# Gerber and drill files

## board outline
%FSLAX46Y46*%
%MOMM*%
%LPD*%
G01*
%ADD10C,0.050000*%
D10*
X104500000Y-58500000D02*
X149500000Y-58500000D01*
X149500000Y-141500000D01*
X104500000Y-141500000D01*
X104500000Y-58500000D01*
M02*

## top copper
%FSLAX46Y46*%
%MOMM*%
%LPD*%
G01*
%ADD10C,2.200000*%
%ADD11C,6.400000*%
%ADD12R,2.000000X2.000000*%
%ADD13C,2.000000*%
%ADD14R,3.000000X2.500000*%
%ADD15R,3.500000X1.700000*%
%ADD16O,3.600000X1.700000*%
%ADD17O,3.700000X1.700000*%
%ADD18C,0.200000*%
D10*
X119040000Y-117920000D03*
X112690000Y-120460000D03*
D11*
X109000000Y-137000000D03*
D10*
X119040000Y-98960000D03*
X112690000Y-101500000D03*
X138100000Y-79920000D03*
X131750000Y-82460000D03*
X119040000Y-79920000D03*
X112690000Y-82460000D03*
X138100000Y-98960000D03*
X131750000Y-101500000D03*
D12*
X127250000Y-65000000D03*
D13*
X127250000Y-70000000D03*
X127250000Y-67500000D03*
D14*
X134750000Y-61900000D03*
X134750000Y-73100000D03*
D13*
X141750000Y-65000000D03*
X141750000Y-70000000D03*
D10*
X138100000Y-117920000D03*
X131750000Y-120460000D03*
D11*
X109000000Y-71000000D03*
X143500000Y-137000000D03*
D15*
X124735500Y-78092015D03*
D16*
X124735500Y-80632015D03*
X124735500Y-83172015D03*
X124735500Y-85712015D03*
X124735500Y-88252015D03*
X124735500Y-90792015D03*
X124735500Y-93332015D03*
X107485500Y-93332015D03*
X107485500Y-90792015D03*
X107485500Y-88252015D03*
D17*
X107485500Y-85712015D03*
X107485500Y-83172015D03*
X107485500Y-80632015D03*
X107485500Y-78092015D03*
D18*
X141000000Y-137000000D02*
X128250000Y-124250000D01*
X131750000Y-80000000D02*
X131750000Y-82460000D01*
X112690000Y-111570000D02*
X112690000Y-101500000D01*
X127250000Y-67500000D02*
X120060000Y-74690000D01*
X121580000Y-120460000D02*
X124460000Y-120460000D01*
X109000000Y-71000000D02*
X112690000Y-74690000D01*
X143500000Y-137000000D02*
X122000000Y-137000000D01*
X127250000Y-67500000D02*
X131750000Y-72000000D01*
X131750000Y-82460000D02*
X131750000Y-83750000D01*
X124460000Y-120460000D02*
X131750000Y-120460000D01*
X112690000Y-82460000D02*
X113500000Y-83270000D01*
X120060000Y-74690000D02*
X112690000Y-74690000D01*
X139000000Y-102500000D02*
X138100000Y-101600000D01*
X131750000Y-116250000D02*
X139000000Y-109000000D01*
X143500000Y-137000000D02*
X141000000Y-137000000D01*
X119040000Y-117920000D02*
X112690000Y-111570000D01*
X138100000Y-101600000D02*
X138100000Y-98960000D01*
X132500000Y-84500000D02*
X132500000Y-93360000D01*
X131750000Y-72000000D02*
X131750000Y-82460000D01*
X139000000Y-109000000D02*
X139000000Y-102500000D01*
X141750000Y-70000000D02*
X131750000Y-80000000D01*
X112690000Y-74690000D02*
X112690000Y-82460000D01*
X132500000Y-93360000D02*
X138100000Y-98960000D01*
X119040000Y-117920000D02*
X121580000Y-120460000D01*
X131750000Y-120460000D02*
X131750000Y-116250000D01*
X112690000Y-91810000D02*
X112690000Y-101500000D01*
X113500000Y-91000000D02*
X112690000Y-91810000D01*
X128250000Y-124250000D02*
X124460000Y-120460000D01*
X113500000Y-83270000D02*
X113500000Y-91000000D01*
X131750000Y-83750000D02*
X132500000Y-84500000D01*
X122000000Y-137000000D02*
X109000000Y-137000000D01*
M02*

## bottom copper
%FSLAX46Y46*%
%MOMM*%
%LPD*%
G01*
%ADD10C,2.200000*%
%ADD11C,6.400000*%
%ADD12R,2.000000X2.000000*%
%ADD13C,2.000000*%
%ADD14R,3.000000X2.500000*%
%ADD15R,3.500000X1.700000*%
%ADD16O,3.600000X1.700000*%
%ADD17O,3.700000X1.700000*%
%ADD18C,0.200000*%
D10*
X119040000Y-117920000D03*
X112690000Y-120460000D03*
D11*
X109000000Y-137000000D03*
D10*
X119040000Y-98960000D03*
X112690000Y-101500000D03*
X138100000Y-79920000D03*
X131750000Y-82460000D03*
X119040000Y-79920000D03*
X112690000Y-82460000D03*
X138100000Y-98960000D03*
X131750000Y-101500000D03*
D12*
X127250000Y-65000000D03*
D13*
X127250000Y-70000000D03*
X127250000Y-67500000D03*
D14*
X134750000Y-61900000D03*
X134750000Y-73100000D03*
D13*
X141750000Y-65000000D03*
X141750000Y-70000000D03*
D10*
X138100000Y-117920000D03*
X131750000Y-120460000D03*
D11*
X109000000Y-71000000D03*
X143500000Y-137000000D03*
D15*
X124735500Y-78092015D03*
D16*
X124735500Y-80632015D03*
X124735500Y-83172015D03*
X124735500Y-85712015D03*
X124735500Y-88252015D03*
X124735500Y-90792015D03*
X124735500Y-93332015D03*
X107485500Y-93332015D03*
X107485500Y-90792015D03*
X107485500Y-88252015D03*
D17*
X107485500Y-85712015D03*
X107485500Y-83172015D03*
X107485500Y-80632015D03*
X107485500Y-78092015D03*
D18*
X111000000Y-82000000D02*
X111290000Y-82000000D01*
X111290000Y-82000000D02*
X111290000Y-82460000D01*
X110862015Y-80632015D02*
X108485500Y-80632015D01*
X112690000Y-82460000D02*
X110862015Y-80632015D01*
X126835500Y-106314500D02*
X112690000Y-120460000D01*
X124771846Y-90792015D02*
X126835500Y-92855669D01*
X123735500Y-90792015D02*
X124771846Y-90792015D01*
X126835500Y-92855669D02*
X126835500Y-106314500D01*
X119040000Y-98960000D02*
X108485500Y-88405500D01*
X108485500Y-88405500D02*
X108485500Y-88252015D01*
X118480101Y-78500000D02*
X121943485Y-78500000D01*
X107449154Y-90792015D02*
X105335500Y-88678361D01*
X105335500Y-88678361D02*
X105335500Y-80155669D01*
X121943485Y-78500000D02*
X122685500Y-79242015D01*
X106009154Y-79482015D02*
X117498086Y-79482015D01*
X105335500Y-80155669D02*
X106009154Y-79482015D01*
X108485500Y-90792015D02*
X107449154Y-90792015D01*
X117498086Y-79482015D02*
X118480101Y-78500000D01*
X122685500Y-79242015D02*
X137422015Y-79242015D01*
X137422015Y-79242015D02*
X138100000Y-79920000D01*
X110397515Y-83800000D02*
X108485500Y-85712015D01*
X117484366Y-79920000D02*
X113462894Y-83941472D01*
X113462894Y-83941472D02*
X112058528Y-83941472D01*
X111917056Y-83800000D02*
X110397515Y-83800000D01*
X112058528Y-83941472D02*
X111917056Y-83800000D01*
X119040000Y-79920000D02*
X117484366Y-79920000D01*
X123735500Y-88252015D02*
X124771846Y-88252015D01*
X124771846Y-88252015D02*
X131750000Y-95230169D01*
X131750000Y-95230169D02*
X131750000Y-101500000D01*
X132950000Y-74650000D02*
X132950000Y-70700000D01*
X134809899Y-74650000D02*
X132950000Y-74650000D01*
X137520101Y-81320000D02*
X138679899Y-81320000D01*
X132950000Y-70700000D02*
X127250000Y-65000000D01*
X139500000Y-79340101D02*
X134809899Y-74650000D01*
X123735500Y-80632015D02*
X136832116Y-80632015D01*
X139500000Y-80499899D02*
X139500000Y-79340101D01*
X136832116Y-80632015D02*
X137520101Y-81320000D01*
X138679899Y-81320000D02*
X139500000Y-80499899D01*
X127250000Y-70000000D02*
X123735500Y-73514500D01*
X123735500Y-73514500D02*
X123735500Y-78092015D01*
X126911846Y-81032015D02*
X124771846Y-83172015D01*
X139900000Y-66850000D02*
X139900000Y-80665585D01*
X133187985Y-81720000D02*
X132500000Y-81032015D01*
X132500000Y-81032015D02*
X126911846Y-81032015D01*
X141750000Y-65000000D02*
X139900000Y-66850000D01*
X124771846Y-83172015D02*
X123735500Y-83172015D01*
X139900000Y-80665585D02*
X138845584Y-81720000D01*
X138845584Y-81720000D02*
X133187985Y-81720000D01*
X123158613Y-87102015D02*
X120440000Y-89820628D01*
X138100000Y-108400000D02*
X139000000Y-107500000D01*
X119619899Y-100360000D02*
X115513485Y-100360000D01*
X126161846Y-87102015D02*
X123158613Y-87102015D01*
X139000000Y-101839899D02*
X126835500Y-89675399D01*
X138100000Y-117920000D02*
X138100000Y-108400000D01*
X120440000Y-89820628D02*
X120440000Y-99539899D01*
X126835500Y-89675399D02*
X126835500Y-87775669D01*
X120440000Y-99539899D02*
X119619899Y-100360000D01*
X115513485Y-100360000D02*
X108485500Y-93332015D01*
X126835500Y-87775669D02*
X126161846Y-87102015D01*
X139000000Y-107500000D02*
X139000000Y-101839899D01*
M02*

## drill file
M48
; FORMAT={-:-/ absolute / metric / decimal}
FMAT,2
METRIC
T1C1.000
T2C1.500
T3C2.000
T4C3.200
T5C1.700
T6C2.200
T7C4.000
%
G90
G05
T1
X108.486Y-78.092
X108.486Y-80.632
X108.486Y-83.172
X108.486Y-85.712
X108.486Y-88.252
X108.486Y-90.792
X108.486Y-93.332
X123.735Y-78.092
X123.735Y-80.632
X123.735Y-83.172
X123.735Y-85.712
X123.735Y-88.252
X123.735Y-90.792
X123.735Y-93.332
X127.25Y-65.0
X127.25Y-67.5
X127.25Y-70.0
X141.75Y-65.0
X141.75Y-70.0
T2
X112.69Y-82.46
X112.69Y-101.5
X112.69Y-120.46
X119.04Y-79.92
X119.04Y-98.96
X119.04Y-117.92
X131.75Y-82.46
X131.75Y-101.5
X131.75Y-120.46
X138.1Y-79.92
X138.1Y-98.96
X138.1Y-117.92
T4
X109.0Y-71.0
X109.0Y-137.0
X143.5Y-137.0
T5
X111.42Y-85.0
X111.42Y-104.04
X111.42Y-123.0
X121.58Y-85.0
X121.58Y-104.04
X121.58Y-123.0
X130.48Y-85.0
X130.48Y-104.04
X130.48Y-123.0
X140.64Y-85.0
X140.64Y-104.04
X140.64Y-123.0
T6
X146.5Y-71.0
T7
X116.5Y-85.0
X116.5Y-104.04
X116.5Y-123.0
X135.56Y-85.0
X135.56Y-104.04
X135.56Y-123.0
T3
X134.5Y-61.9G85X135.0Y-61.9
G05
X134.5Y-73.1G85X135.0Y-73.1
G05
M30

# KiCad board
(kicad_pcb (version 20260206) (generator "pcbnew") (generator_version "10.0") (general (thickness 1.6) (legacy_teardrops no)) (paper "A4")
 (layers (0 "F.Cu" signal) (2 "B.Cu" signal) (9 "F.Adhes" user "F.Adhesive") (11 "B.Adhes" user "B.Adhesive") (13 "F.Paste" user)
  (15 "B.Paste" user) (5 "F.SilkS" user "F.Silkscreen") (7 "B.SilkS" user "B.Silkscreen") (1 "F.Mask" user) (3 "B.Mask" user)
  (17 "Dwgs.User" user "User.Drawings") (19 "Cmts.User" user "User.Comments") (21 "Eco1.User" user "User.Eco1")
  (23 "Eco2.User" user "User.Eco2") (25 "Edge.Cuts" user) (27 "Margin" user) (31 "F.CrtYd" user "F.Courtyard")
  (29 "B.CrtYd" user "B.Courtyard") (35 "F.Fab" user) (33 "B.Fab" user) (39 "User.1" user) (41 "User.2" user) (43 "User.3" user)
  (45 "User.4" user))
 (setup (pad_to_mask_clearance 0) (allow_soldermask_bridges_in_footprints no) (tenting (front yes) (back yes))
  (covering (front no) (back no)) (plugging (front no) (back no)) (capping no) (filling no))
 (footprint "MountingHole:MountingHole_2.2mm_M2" (layer "F.Cu") (at 146.5 71)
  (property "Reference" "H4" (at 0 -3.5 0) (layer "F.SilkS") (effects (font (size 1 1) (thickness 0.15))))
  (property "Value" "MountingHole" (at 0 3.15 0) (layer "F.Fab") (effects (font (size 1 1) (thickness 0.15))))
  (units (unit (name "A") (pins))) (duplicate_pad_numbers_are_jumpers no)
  (pad "" np_thru_hole circle (at 0 0) (size 2.2 2.2) (drill 2.2) (layers "*.Cu" "*.Mask")))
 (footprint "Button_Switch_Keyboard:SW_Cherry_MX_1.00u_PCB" (layer "F.Cu") (at 119.04 117.92)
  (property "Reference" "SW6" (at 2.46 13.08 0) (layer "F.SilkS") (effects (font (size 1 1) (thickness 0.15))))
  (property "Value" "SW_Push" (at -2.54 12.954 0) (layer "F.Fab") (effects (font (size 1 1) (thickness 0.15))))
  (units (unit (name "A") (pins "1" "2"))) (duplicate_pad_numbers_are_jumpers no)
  (pad "" np_thru_hole circle (at -7.62 5.08) (size 1.7 1.7) (drill 1.7) (layers "*.Cu" "*.Mask"))
  (pad "" np_thru_hole circle (at -2.54 5.08) (size 4 4) (drill 4) (layers "*.Cu" "*.Mask"))
  (pad "" np_thru_hole circle (at 2.54 5.08) (size 1.7 1.7) (drill 1.7) (layers "*.Cu" "*.Mask"))
  (pad "1" thru_hole circle (at 0 0) (size 2.2 2.2) (drill 1.5) (layers "*.Cu" "*.Mask") (remove_unused_layers no) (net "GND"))
  (pad "2" thru_hole circle (at -6.35 2.54) (size 2.2 2.2) (drill 1.5) (layers "*.Cu" "*.Mask") (remove_unused_layers no)
   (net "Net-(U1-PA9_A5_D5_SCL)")))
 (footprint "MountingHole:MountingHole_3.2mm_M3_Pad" (layer "F.Cu") (at 109 137)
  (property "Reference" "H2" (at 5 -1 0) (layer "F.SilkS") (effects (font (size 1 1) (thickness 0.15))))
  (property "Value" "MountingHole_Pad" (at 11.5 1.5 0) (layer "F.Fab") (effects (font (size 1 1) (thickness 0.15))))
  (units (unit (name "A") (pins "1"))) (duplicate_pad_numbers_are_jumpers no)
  (pad "1" thru_hole circle (at 0 0) (size 6.4 6.4) (drill 3.2) (layers "*.Cu" "*.Mask") (remove_unused_layers no) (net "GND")
   (zone_connect 2)))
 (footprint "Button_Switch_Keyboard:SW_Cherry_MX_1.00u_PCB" (layer "F.Cu") (at 119.04 98.96)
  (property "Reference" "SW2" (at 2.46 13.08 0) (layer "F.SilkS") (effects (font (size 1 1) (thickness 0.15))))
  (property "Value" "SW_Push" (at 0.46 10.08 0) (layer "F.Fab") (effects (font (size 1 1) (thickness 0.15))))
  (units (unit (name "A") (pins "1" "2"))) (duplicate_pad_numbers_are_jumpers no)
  (pad "" np_thru_hole circle (at -7.62 5.08) (size 1.7 1.7) (drill 1.7) (layers "*.Cu" "*.Mask"))
  (pad "" np_thru_hole circle (at -2.54 5.08) (size 4 4) (drill 4) (layers "*.Cu" "*.Mask"))
  (pad "" np_thru_hole circle (at 2.54 5.08) (size 1.7 1.7) (drill 1.7) (layers "*.Cu" "*.Mask"))
  (pad "1" thru_hole circle (at 0 0) (size 2.2 2.2) (drill 1.5) (layers "*.Cu" "*.Mask") (remove_unused_layers no)
   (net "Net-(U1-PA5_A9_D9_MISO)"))
  (pad "2" thru_hole circle (at -6.35 2.54) (size 2.2 2.2) (drill 1.5) (layers "*.Cu" "*.Mask") (remove_unused_layers no) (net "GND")))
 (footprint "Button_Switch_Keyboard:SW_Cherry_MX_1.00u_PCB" (layer "F.Cu") (at 138.1 79.92)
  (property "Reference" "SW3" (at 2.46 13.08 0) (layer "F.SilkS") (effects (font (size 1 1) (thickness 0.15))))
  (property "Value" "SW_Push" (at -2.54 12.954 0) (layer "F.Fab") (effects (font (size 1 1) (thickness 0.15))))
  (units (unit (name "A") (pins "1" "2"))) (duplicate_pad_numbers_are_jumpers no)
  (pad "" np_thru_hole circle (at -7.62 5.08) (size 1.7 1.7) (drill 1.7) (layers "*.Cu" "*.Mask"))
  (pad "" np_thru_hole circle (at -2.54 5.08) (size 4 4) (drill 4) (layers "*.Cu" "*.Mask"))
  (pad "" np_thru_hole circle (at 2.54 5.08) (size 1.7 1.7) (drill 1.7) (layers "*.Cu" "*.Mask"))
  (pad "1" thru_hole circle (at 0 0) (size 2.2 2.2) (drill 1.5) (layers "*.Cu" "*.Mask") (remove_unused_layers no)
   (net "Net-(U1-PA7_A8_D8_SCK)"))
  (pad "2" thru_hole circle (at -6.35 2.54) (size 2.2 2.2) (drill 1.5) (layers "*.Cu" "*.Mask") (remove_unused_layers no) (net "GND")))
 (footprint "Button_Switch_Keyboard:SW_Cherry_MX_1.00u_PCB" (layer "F.Cu") (at 119.04 79.92)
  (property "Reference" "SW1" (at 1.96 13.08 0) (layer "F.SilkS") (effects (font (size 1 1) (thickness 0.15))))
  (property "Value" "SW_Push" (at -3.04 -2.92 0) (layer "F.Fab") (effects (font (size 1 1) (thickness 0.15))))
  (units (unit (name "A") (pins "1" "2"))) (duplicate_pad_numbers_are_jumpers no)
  (pad "" np_thru_hole circle (at -7.62 5.08) (size 1.7 1.7) (drill 1.7) (layers "*.Cu" "*.Mask"))
  (pad "" np_thru_hole circle (at -2.54 5.08) (size 4 4) (drill 4) (layers "*.Cu" "*.Mask"))
  (pad "" np_thru_hole circle (at 2.54 5.08) (size 1.7 1.7) (drill 1.7) (layers "*.Cu" "*.Mask"))
  (pad "1" thru_hole circle (at 0 0) (size 2.2 2.2) (drill 1.5) (layers "*.Cu" "*.Mask") (remove_unused_layers no)
   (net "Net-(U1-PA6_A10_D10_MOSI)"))
  (pad "2" thru_hole circle (at -6.35 2.54) (size 2.2 2.2) (drill 1.5) (layers "*.Cu" "*.Mask") (remove_unused_layers no) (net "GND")))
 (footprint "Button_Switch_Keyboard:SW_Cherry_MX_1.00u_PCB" (layer "F.Cu") (at 138.1 98.96)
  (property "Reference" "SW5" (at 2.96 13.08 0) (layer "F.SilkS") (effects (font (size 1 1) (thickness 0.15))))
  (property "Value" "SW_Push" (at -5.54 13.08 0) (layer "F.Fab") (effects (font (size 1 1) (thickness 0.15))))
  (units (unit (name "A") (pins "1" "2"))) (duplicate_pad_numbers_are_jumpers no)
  (pad "" np_thru_hole circle (at -7.62 5.08) (size 1.7 1.7) (drill 1.7) (layers "*.Cu" "*.Mask"))
  (pad "" np_thru_hole circle (at -2.54 5.08) (size 4 4) (drill 4) (layers "*.Cu" "*.Mask"))
  (pad "" np_thru_hole circle (at 2.54 5.08) (size 1.7 1.7) (drill 1.7) (layers "*.Cu" "*.Mask"))
  (pad "1" thru_hole circle (at 0 0) (size 2.2 2.2) (drill 1.5) (layers "*.Cu" "*.Mask") (remove_unused_layers no) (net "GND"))
  (pad "2" thru_hole circle (at -6.35 2.54) (size 2.2 2.2) (drill 1.5) (layers "*.Cu" "*.Mask") (remove_unused_layers no)
   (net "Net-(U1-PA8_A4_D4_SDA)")))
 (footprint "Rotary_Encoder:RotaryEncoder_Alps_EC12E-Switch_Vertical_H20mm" (layer "F.Cu") (at 127.25 65)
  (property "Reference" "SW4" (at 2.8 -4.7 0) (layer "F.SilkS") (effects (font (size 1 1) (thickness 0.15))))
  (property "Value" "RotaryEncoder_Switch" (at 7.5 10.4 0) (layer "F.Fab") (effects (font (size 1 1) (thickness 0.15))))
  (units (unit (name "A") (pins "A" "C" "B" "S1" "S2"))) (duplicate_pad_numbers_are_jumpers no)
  (pad "A" thru_hole rect (at 0 0) (size 2 2) (drill 1) (layers "*.Cu" "*.Mask") (remove_unused_layers no) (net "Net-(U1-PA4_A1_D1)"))
  (pad "B" thru_hole circle (at 0 5) (size 2 2) (drill 1) (layers "*.Cu" "*.Mask") (remove_unused_layers no) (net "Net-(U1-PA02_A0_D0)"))
  (pad "C" thru_hole circle (at 0 2.5) (size 2 2) (drill 1) (layers "*.Cu" "*.Mask") (remove_unused_layers no) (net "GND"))
  (pad "MP" thru_hole rect (at 7.5 -3.1) (size 3 2.5) (drill oval 2.5 2) (layers "*.Cu" "*.Mask") (remove_unused_layers no))
  (pad "MP" thru_hole rect (at 7.5 8.1) (size 3 2.5) (drill oval 2.5 2) (layers "*.Cu" "*.Mask") (remove_unused_layers no))
  (pad "S1" thru_hole circle (at 14.5 0) (size 2 2) (drill 1) (layers "*.Cu" "*.Mask") (remove_unused_layers no) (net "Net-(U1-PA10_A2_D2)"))
  (pad "S2" thru_hole circle (at 14.5 5) (size 2 2) (drill 1) (layers "*.Cu" "*.Mask") (remove_unused_layers no) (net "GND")))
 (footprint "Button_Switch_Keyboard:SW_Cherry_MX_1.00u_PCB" (layer "F.Cu") (at 138.1 117.92)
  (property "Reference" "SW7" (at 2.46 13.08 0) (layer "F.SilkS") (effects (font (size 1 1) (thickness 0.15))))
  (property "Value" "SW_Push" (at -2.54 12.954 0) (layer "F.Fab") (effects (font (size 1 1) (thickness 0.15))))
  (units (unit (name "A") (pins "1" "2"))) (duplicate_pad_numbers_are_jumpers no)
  (pad "" np_thru_hole circle (at -7.62 5.08) (size 1.7 1.7) (drill 1.7) (layers "*.Cu" "*.Mask"))
  (pad "" np_thru_hole circle (at -2.54 5.08) (size 4 4) (drill 4) (layers "*.Cu" "*.Mask"))
  (pad "" np_thru_hole circle (at 2.54 5.08) (size 1.7 1.7) (drill 1.7) (layers "*.Cu" "*.Mask"))
  (pad "1" thru_hole circle (at 0 0) (size 2.2 2.2) (drill 1.5) (layers "*.Cu" "*.Mask") (remove_unused_layers no)
   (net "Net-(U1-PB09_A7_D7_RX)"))
  (pad "2" thru_hole circle (at -6.35 2.54) (size 2.2 2.2) (drill 1.5) (layers "*.Cu" "*.Mask") (remove_unused_layers no) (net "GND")))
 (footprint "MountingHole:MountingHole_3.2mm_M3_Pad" (layer "F.Cu") (at 109 71)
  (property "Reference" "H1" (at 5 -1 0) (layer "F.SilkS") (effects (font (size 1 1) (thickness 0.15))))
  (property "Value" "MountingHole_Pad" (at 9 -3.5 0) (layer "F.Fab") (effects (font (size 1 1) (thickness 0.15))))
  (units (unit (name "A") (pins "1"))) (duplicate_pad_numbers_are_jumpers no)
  (pad "1" thru_hole circle (at 0 0) (size 6.4 6.4) (drill 3.2) (layers "*.Cu" "*.Mask") (remove_unused_layers no) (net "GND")
   (zone_connect 2)))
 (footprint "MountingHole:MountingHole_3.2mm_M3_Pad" (layer "F.Cu") (at 143.5 137)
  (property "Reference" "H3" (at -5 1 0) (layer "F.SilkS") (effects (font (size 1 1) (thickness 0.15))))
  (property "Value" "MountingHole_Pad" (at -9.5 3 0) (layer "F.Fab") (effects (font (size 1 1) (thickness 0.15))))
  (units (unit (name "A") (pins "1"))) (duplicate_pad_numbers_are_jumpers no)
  (pad "1" thru_hole circle (at 0 0) (size 6.4 6.4) (drill 3.2) (layers "*.Cu" "*.Mask") (remove_unused_layers no) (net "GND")
   (zone_connect 2)))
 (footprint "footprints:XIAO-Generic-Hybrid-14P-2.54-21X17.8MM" (layer "B.Cu") (at 116.1105 85.712015 180)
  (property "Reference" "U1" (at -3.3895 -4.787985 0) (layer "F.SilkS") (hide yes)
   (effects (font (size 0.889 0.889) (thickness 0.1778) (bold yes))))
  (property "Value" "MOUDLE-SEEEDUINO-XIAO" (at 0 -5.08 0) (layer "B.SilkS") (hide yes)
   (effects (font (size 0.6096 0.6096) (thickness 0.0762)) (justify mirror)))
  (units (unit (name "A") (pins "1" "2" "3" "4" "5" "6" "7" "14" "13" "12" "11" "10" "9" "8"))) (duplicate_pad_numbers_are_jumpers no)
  (pad "1" thru_hole rect (at -7.625 7.62 180) (size 3.5 1.7) (drill 1 (offset -1 0)) (layers "*.Cu" "*.Mask") (remove_unused_layers no)
   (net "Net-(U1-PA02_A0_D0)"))
  (pad "2" thru_hole oval (at -7.625 5.08 180) (size 3.6 1.7) (drill 1 (offset -1 0)) (layers "*.Cu" "*.Mask") (remove_unused_layers no)
   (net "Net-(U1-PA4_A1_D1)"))
  (pad "3" thru_hole oval (at -7.625 2.54 180) (size 3.6 1.7) (drill 1 (offset -1 0)) (layers "*.Cu" "*.Mask") (remove_unused_layers no)
   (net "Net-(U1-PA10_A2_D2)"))
  (pad "4" thru_hole oval (at -7.625 0 180) (size 3.6 1.7) (drill 1 (offset -1 0)) (layers "*.Cu" "*.Mask") (remove_unused_layers no)
   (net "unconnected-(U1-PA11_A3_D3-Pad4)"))
  (pad "5" thru_hole oval (at -7.625 -2.54 180) (size 3.6 1.7) (drill 1 (offset -1 0)) (layers "*.Cu" "*.Mask") (remove_unused_layers no)
   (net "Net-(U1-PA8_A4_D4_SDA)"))
  (pad "6" thru_hole oval (at -7.625 -5.08) (size 3.6 1.7) (drill 1 (offset 1 0)) (layers "*.Cu" "*.Mask") (remove_unused_layers no)
   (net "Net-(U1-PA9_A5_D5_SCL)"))
  (pad "7" thru_hole oval (at -7.625 -7.62 180) (size 3.6 1.7) (drill 1 (offset -1 0)) (layers "*.Cu" "*.Mask") (remove_unused_layers no)
   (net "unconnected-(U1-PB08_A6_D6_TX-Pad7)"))
  (pad "8" thru_hole oval (at 7.625 -7.62 180) (size 3.6 1.7) (drill 1 (offset 1 0)) (layers "*.Cu" "*.Mask") (remove_unused_layers no)
   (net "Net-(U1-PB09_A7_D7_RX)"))
  (pad "9" thru_hole oval (at 7.625 -5.08 180) (size 3.6 1.7) (drill 1 (offset 1 0)) (layers "*.Cu" "*.Mask") (remove_unused_layers no)
   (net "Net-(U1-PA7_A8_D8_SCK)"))
  (pad "10" thru_hole oval (at 7.625 -2.54 180) (size 3.6 1.7) (drill 1 (offset 1 0)) (layers "*.Cu" "*.Mask") (remove_unused_layers no)
   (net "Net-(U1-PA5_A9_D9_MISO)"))
  (pad "11" thru_hole oval (at 7.625 0 180) (size 3.7 1.7) (drill 1 (offset 1 0)) (layers "*.Cu" "*.Mask") (remove_unused_layers no)
   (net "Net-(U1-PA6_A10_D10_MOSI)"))
  (pad "12" thru_hole oval (at 7.625 2.54 180) (size 3.7 1.7) (drill 1 (offset 1 0)) (layers "*.Cu" "*.Mask") (remove_unused_layers no)
   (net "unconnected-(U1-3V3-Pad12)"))
  (pad "13" thru_hole oval (at 7.625 5.08 180) (size 3.7 1.7) (drill 1 (offset 1 0)) (layers "*.Cu" "*.Mask") (remove_unused_layers no)
   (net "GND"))
  (pad "14" thru_hole oval (at 7.625 7.62 180) (size 3.7 1.7) (drill 1 (offset 1 0)) (layers "*.Cu" "*.Mask") (remove_unused_layers no)
   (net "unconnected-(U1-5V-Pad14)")))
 (gr_rect (start 104.5 58.5) (end 149.5 141.5) (stroke (width 0.05) (type default)) (fill no) (layer "Edge.Cuts"))
 (segment (start 111 82) (end 111.29 82) (width 0.2) (layer "B.Cu") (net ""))
 (segment (start 111.29 82) (end 111.29 82.46) (width 0.2) (layer "B.Cu") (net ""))
 (segment (start 141 137) (end 128.25 124.25) (width 0.2) (layer "F.Cu") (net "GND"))
 (segment (start 131.75 80) (end 131.75 82.46) (width 0.2) (layer "F.Cu") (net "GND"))
 (segment (start 112.69 111.57) (end 112.69 101.5) (width 0.2) (layer "F.Cu") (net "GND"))
 (segment (start 127.25 67.5) (end 120.06 74.69) (width 0.2) (layer "F.Cu") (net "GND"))
 (segment (start 121.58 120.46) (end 124.46 120.46) (width 0.2) (layer "F.Cu") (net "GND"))
 (segment (start 109 71) (end 112.69 74.69) (width 0.2) (layer "F.Cu") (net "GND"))
 (segment (start 143.5 137) (end 122 137) (width 0.2) (layer "F.Cu") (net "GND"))
 (segment (start 127.25 67.5) (end 131.75 72) (width 0.2) (layer "F.Cu") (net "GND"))
 (segment (start 131.75 82.46) (end 131.75 83.75) (width 0.2) (layer "F.Cu") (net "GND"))
 (segment (start 124.46 120.46) (end 131.75 120.46) (width 0.2) (layer "F.Cu") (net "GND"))
 (segment (start 112.69 82.46) (end 113.5 83.27) (width 0.2) (layer "F.Cu") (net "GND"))
 (segment (start 120.06 74.69) (end 112.69 74.69) (width 0.2) (layer "F.Cu") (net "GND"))
 (segment (start 139 102.5) (end 138.1 101.6) (width 0.2) (layer "F.Cu") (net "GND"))
 (segment (start 131.75 116.25) (end 139 109) (width 0.2) (layer "F.Cu") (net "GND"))
 (segment (start 143.5 137) (end 141 137) (width 0.2) (layer "F.Cu") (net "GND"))
 (segment (start 119.04 117.92) (end 112.69 111.57) (width 0.2) (layer "F.Cu") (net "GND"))
 (segment (start 138.1 101.6) (end 138.1 98.96) (width 0.2) (layer "F.Cu") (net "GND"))
 (segment (start 132.5 84.5) (end 132.5 93.36) (width 0.2) (layer "F.Cu") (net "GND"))
 (segment (start 131.75 72) (end 131.75 82.46) (width 0.2) (layer "F.Cu") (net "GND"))
 (segment (start 139 109) (end 139 102.5) (width 0.2) (layer "F.Cu") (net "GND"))
 (segment (start 141.75 70) (end 131.75 80) (width 0.2) (layer "F.Cu") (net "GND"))
 (segment (start 112.69 74.69) (end 112.69 82.46) (width 0.2) (layer "F.Cu") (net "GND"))
 (segment (start 132.5 93.36) (end 138.1 98.96) (width 0.2) (layer "F.Cu") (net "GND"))
 (segment (start 119.04 117.92) (end 121.58 120.46) (width 0.2) (layer "F.Cu") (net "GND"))
 (segment (start 131.75 120.46) (end 131.75 116.25) (width 0.2) (layer "F.Cu") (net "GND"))
 (segment (start 112.69 91.81) (end 112.69 101.5) (width 0.2) (layer "F.Cu") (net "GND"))
 (segment (start 113.5 91) (end 112.69 91.81) (width 0.2) (layer "F.Cu") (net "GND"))
 (segment (start 128.25 124.25) (end 124.46 120.46) (width 0.2) (layer "F.Cu") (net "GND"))
 (segment (start 113.5 83.27) (end 113.5 91) (width 0.2) (layer "F.Cu") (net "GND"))
 (segment (start 131.75 83.75) (end 132.5 84.5) (width 0.2) (layer "F.Cu") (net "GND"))
 (segment (start 122 137) (end 109 137) (width 0.2) (layer "F.Cu") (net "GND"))
 (segment (start 110.862015 80.632015) (end 108.4855 80.632015) (width 0.2) (layer "B.Cu") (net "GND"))
 (segment (start 112.69 82.46) (end 110.862015 80.632015) (width 0.2) (layer "B.Cu") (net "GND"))
 (segment (start 126.8355 106.3145) (end 112.69 120.46) (width 0.2) (layer "B.Cu") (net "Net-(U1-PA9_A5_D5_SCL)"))
 (segment (start 124.771846 90.792015) (end 126.8355 92.855669) (width 0.2) (layer "B.Cu") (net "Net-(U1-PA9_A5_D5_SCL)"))
 (segment (start 123.7355 90.792015) (end 124.771846 90.792015) (width 0.2) (layer "B.Cu") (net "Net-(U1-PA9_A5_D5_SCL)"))
 (segment (start 126.8355 92.855669) (end 126.8355 106.3145) (width 0.2) (layer "B.Cu") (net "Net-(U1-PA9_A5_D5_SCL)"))
 (segment (start 119.04 98.96) (end 108.4855 88.4055) (width 0.2) (layer "B.Cu") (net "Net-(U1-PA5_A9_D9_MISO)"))
 (segment (start 108.4855 88.4055) (end 108.4855 88.252015) (width 0.2) (layer "B.Cu") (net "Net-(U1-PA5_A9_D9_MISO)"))
 (segment (start 118.480101 78.5) (end 121.943485 78.5) (width 0.2) (layer "B.Cu") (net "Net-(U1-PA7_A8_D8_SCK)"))
 (segment (start 107.449154 90.792015) (end 105.3355 88.678361) (width 0.2) (layer "B.Cu") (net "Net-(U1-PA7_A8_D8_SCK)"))
 (segment (start 105.3355 88.678361) (end 105.3355 80.155669) (width 0.2) (layer "B.Cu") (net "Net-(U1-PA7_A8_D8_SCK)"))
 (segment (start 121.943485 78.5) (end 122.6855 79.242015) (width 0.2) (layer "B.Cu") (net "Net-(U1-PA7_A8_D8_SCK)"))
 (segment (start 106.009154 79.482015) (end 117.498086 79.482015) (width 0.2) (layer "B.Cu") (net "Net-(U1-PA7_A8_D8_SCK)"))
 (segment (start 105.3355 80.155669) (end 106.009154 79.482015) (width 0.2) (layer "B.Cu") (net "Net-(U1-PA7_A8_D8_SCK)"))
 (segment (start 108.4855 90.792015) (end 107.449154 90.792015) (width 0.2) (layer "B.Cu") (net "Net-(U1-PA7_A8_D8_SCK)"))
 (segment (start 117.498086 79.482015) (end 118.480101 78.5) (width 0.2) (layer "B.Cu") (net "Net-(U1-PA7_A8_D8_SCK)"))
 (segment (start 122.6855 79.242015) (end 137.422015 79.242015) (width 0.2) (layer "B.Cu") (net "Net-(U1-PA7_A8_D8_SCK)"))
 (segment (start 137.422015 79.242015) (end 138.1 79.92) (width 0.2) (layer "B.Cu") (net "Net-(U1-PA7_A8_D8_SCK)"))
 (segment (start 110.397515 83.8) (end 108.4855 85.712015) (width 0.2) (layer "B.Cu") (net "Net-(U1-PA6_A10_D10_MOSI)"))
 (segment (start 117.484366 79.92) (end 113.462894 83.941472) (width 0.2) (layer "B.Cu") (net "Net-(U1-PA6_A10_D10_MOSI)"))
 (segment (start 113.462894 83.941472) (end 112.058528 83.941472) (width 0.2) (layer "B.Cu") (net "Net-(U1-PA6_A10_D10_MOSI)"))
 (segment (start 111.917056 83.8) (end 110.397515 83.8) (width 0.2) (layer "B.Cu") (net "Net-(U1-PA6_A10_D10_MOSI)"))
 (segment (start 112.058528 83.941472) (end 111.917056 83.8) (width 0.2) (layer "B.Cu") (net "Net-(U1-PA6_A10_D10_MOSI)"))
 (segment (start 119.04 79.92) (end 117.484366 79.92) (width 0.2) (layer "B.Cu") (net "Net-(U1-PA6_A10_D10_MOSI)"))
 (segment (start 123.7355 88.252015) (end 124.771846 88.252015) (width 0.2) (layer "B.Cu") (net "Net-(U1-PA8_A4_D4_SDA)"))
 (segment (start 124.771846 88.252015) (end 131.75 95.230169) (width 0.2) (layer "B.Cu") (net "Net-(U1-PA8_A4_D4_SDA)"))
 (segment (start 131.75 95.230169) (end 131.75 101.5) (width 0.2) (layer "B.Cu") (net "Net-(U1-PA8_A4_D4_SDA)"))
 (segment (start 132.95 74.65) (end 132.95 70.7) (width 0.2) (layer "B.Cu") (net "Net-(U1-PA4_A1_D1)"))
 (segment (start 134.809899 74.65) (end 132.95 74.65) (width 0.2) (layer "B.Cu") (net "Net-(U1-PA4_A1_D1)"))
 (segment (start 137.520101 81.32) (end 138.679899 81.32) (width 0.2) (layer "B.Cu") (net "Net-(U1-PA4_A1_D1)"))
 (segment (start 132.95 70.7) (end 127.25 65) (width 0.2) (layer "B.Cu") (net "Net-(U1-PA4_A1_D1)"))
 (segment (start 139.5 79.340101) (end 134.809899 74.65) (width 0.2) (layer "B.Cu") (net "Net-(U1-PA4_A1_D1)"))
 (segment (start 123.7355 80.632015) (end 136.832116 80.632015) (width 0.2) (layer "B.Cu") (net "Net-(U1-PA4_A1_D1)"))
 (segment (start 139.5 80.499899) (end 139.5 79.340101) (width 0.2) (layer "B.Cu") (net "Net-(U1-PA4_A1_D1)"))
 (segment (start 136.832116 80.632015) (end 137.520101 81.32) (width 0.2) (layer "B.Cu") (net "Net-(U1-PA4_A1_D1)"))
 (segment (start 138.679899 81.32) (end 139.5 80.499899) (width 0.2) (layer "B.Cu") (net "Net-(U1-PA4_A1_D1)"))
 (segment (start 127.25 70) (end 123.7355 73.5145) (width 0.2) (layer "B.Cu") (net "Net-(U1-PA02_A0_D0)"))
 (segment (start 123.7355 73.5145) (end 123.7355 78.092015) (width 0.2) (layer "B.Cu") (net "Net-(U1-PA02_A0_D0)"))
 (segment (start 126.911846 81.032015) (end 124.771846 83.172015) (width 0.2) (layer "B.Cu") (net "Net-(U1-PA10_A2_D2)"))
 (segment (start 139.9 66.85) (end 139.9 80.665585) (width 0.2) (layer "B.Cu") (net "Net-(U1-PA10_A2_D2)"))
 (segment (start 133.187985 81.72) (end 132.5 81.032015) (width 0.2) (layer "B.Cu") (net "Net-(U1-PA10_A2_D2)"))
 (segment (start 132.5 81.032015) (end 126.911846 81.032015) (width 0.2) (layer "B.Cu") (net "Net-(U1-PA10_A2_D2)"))
 (segment (start 141.75 65) (end 139.9 66.85) (width 0.2) (layer "B.Cu") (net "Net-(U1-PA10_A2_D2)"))
 (segment (start 124.771846 83.172015) (end 123.7355 83.172015) (width 0.2) (layer "B.Cu") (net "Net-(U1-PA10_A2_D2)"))
 (segment (start 139.9 80.665585) (end 138.845584 81.72) (width 0.2) (layer "B.Cu") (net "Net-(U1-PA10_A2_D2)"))
 (segment (start 138.845584 81.72) (end 133.187985 81.72) (width 0.2) (layer "B.Cu") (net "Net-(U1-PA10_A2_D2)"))
 (segment (start 123.158613 87.102015) (end 120.44 89.820628) (width 0.2) (layer "B.Cu") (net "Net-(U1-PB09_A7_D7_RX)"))
 (segment (start 138.1 108.4) (end 139 107.5) (width 0.2) (layer "B.Cu") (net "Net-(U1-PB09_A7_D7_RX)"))
 (segment (start 119.619899 100.36) (end 115.513485 100.36) (width 0.2) (layer "B.Cu") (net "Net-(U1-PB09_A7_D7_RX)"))
 (segment (start 126.161846 87.102015) (end 123.158613 87.102015) (width 0.2) (layer "B.Cu") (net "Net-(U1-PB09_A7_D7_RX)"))
 (segment (start 139 101.839899) (end 126.8355 89.675399) (width 0.2) (layer "B.Cu") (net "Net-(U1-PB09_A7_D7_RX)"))
 (segment (start 138.1 117.92) (end 138.1 108.4) (width 0.2) (layer "B.Cu") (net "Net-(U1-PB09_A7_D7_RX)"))
 (segment (start 120.44 89.820628) (end 120.44 99.539899) (width 0.2) (layer "B.Cu") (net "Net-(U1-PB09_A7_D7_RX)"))
 (segment (start 126.8355 89.675399) (end 126.8355 87.775669) (width 0.2) (layer "B.Cu") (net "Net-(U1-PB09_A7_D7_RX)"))
 (segment (start 120.44 99.539899) (end 119.619899 100.36) (width 0.2) (layer "B.Cu") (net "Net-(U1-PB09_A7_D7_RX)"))
 (segment (start 115.513485 100.36) (end 108.4855 93.332015) (width 0.2) (layer "B.Cu") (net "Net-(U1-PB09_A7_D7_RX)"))
 (segment (start 126.8355 87.775669) (end 126.161846 87.102015) (width 0.2) (layer "B.Cu") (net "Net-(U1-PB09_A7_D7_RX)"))
 (segment (start 139 107.5) (end 139 101.839899) (width 0.2) (layer "B.Cu") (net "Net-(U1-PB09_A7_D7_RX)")))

